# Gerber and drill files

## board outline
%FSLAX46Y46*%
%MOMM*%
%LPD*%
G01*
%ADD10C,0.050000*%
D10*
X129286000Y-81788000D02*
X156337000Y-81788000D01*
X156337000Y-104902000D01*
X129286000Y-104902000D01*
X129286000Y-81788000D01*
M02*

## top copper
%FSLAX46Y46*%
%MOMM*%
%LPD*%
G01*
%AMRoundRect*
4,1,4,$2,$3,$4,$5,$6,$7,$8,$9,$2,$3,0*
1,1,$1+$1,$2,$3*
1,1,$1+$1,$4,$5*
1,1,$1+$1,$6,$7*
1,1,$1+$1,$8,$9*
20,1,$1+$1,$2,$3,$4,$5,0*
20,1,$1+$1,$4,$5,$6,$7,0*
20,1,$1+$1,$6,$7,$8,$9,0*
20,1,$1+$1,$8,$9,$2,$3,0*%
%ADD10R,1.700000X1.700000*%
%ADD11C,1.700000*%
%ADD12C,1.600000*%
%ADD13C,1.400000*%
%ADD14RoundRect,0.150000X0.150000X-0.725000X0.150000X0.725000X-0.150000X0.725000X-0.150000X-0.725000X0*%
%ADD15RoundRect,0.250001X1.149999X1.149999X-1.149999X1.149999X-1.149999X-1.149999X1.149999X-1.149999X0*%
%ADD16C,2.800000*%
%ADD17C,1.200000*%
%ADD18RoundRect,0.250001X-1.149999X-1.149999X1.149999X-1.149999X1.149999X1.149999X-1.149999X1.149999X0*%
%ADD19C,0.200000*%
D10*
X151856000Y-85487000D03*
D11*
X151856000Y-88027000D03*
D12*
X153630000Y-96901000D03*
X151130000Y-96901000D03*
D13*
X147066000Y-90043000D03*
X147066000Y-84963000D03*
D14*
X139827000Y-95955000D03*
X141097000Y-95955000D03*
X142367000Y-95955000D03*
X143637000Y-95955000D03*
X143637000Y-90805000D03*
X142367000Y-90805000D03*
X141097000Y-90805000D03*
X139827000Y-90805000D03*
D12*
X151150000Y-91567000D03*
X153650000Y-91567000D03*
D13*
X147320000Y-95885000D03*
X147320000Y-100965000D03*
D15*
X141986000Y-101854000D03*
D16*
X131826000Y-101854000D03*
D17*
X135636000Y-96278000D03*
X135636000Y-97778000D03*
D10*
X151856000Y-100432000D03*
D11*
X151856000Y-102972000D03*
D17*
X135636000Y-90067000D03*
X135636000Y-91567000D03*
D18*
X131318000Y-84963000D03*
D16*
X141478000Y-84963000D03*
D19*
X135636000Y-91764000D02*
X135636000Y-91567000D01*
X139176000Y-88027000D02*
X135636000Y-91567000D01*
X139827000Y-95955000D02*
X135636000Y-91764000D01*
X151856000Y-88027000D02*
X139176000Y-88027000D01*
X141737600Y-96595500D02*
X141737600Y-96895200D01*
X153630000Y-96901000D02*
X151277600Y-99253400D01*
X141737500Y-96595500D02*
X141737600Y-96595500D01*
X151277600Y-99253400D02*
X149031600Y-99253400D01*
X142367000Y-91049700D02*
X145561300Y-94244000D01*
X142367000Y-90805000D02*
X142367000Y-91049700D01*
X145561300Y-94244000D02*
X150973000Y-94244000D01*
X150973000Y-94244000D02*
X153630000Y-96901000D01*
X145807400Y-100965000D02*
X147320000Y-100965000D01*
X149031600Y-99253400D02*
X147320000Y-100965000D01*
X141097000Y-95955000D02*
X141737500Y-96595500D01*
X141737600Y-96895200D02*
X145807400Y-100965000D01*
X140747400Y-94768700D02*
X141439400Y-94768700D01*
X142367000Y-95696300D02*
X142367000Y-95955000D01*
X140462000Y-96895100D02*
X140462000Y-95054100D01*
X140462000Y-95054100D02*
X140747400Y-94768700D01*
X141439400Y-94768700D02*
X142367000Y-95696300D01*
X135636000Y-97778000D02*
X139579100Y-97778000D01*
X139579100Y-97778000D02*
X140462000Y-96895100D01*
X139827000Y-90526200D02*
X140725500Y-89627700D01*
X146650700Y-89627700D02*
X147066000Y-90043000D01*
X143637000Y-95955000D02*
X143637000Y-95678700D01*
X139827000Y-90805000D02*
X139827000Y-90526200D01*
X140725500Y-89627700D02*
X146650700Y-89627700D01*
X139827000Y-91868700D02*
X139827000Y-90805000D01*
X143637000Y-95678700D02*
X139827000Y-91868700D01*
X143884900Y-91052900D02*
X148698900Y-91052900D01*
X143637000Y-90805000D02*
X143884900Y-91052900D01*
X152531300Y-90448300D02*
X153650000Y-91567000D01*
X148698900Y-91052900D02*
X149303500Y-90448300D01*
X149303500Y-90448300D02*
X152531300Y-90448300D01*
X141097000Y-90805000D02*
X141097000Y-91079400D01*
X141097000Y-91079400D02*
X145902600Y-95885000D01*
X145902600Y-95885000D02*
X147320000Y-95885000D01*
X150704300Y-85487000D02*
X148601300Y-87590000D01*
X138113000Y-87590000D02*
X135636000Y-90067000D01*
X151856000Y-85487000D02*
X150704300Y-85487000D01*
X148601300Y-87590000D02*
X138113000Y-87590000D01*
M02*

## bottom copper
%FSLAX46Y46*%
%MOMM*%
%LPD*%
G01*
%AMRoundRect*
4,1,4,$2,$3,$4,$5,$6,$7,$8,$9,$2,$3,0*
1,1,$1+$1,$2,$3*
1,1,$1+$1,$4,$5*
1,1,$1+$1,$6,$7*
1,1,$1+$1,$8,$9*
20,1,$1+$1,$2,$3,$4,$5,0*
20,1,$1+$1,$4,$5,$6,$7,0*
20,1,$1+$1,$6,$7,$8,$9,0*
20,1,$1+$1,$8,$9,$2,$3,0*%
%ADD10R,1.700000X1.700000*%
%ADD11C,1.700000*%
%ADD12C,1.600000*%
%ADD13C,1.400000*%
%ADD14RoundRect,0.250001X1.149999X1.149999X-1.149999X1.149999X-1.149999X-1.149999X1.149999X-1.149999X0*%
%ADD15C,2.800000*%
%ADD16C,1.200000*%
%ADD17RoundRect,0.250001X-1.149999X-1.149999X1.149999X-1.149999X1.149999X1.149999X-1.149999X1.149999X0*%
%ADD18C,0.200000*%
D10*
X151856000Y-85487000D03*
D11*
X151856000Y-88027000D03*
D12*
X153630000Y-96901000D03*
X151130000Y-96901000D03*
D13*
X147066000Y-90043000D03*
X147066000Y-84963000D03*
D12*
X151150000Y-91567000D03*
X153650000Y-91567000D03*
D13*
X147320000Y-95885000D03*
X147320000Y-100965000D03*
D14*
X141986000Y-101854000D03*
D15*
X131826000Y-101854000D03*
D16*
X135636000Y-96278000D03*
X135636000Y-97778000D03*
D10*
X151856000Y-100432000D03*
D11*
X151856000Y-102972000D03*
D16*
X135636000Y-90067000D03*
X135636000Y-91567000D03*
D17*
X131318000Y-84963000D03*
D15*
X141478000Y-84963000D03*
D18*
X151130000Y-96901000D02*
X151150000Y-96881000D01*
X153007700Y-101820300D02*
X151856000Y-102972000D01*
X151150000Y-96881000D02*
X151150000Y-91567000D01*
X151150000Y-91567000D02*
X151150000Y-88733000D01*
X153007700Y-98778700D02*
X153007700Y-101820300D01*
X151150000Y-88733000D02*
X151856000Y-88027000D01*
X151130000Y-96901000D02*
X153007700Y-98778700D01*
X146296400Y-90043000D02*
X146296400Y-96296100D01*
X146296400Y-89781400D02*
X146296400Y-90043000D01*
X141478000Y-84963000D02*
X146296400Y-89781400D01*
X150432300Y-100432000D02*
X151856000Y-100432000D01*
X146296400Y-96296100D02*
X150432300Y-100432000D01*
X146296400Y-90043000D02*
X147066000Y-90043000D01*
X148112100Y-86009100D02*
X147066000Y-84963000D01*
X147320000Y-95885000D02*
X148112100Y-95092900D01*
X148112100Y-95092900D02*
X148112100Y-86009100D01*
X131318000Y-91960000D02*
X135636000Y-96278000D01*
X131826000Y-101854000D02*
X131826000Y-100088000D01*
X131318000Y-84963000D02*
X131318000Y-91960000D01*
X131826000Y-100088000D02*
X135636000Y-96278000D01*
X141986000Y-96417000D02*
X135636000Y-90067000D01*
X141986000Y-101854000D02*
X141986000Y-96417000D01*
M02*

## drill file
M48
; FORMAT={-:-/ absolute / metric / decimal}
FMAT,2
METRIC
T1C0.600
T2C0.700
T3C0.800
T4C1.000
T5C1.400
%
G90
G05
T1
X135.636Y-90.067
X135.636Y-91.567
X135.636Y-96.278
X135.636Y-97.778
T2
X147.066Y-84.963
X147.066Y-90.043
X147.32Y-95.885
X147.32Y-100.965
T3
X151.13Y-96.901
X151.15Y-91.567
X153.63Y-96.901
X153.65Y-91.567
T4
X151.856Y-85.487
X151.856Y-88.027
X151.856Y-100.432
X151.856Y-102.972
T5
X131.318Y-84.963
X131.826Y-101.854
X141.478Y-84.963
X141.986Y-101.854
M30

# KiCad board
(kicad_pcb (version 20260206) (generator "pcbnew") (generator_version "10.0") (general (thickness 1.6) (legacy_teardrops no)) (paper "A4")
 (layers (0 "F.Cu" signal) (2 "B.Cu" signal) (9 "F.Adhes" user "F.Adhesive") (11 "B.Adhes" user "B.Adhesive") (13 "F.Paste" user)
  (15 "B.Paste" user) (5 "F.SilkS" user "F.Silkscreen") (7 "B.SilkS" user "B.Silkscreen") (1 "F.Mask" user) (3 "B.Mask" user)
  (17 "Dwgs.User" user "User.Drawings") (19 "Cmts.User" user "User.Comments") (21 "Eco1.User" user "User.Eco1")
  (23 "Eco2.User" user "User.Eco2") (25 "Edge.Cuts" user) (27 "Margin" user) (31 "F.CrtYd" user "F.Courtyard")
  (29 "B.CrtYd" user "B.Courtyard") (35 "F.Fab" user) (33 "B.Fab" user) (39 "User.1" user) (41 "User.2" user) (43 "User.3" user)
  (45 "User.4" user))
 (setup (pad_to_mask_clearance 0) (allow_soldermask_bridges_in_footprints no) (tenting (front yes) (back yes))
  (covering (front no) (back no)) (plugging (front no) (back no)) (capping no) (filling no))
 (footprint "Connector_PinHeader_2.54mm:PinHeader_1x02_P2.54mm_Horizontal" (layer "F.Cu") (at 151.856 85.487)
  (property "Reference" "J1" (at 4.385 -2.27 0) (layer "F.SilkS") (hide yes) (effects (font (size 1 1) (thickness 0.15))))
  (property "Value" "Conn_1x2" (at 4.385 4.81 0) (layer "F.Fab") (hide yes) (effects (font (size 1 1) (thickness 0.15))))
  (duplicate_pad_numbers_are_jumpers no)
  (pad "1" thru_hole rect (at 0 0) (size 1.7 1.7) (drill 1) (layers "*.Cu" "*.Mask") (remove_unused_layers no) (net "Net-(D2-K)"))
  (pad "2" thru_hole circle (at 0 2.54) (size 1.7 1.7) (drill 1) (layers "*.Cu" "*.Mask") (remove_unused_layers no) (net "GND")))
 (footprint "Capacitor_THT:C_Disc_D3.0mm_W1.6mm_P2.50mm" (layer "F.Cu") (at 153.63 96.901 180)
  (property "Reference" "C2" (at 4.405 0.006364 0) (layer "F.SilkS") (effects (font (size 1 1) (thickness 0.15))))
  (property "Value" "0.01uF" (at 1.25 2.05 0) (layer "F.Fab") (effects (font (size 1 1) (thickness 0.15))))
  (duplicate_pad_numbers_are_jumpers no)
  (pad "1" thru_hole circle (at 0 0 180) (size 1.6 1.6) (drill 0.8) (layers "*.Cu" "*.Mask") (remove_unused_layers no)
   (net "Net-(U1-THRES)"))
  (pad "2" thru_hole circle (at 2.5 0 180) (size 1.6 1.6) (drill 0.8) (layers "*.Cu" "*.Mask") (remove_unused_layers no) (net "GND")))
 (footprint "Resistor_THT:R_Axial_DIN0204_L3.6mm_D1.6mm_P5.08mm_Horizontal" (layer "F.Cu") (at 147.066 90.043 90)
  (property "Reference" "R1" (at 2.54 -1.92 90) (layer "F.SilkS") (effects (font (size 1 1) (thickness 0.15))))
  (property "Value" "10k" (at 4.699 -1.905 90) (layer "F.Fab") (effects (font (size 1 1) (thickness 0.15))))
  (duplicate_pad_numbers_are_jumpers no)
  (pad "1" thru_hole circle (at 0 0 90) (size 1.4 1.4) (drill 0.7) (layers "*.Cu" "*.Mask") (remove_unused_layers no) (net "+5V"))
  (pad "2" thru_hole circle (at 5.08 0 90) (size 1.4 1.4) (drill 0.7) (layers "*.Cu" "*.Mask") (remove_unused_layers no)
   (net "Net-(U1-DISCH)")))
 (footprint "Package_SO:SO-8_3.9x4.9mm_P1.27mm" (layer "F.Cu") (at 141.732 93.38 90)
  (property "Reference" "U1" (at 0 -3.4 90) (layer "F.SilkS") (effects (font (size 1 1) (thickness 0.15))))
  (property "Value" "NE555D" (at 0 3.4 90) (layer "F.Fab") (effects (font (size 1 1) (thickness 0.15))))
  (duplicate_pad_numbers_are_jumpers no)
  (pad "1" smd roundrect (at -2.575 -1.905 90) (size 1.75 0.6) (layers "F.Cu" "F.Mask" "F.Paste") (roundrect_rratio 0.25) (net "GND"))
  (pad "2" smd roundrect (at -2.575 -0.635 90) (size 1.75 0.6) (layers "F.Cu" "F.Mask" "F.Paste") (roundrect_rratio 0.25)
   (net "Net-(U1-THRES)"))
  (pad "3" smd roundrect (at -2.575 0.635 90) (size 1.75 0.6) (layers "F.Cu" "F.Mask" "F.Paste") (roundrect_rratio 0.25)
   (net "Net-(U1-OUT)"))
  (pad "4" smd roundrect (at -2.575 1.905 90) (size 1.75 0.6) (layers "F.Cu" "F.Mask" "F.Paste") (roundrect_rratio 0.25) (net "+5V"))
  (pad "5" smd roundrect (at 2.575 1.905 90) (size 1.75 0.6) (layers "F.Cu" "F.Mask" "F.Paste") (roundrect_rratio 0.25)
   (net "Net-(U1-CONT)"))
  (pad "6" smd roundrect (at 2.575 0.635 90) (size 1.75 0.6) (layers "F.Cu" "F.Mask" "F.Paste") (roundrect_rratio 0.25)
   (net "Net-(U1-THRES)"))
  (pad "7" smd roundrect (at 2.575 -0.635 90) (size 1.75 0.6) (layers "F.Cu" "F.Mask" "F.Paste") (roundrect_rratio 0.25)
   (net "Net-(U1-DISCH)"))
  (pad "8" smd roundrect (at 2.575 -1.905 90) (size 1.75 0.6) (layers "F.Cu" "F.Mask" "F.Paste") (roundrect_rratio 0.25) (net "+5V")))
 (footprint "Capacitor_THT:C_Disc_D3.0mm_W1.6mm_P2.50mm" (layer "F.Cu") (at 151.15 91.567)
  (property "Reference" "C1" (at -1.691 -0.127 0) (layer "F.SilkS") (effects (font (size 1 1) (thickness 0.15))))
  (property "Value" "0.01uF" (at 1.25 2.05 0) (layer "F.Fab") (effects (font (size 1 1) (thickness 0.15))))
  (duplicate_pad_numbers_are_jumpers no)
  (pad "1" thru_hole circle (at 0 0) (size 1.6 1.6) (drill 0.8) (layers "*.Cu" "*.Mask") (remove_unused_layers no) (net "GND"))
  (pad "2" thru_hole circle (at 2.5 0) (size 1.6 1.6) (drill 0.8) (layers "*.Cu" "*.Mask") (remove_unused_layers no) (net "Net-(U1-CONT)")))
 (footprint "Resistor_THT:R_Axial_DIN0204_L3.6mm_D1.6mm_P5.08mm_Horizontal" (layer "F.Cu") (at 147.32 95.885 -90)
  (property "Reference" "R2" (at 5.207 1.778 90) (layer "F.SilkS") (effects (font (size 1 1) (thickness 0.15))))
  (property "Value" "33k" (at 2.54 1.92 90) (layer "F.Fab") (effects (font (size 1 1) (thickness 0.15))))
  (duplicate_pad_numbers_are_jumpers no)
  (pad "1" thru_hole circle (at 0 0 270) (size 1.4 1.4) (drill 0.7) (layers "*.Cu" "*.Mask") (remove_unused_layers no)
   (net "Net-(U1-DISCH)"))
  (pad "2" thru_hole circle (at 5.08 0 270) (size 1.4 1.4) (drill 0.7) (layers "*.Cu" "*.Mask") (remove_unused_layers no)
   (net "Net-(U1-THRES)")))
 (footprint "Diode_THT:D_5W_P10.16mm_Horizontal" (layer "F.Cu") (at 141.986 101.854 180)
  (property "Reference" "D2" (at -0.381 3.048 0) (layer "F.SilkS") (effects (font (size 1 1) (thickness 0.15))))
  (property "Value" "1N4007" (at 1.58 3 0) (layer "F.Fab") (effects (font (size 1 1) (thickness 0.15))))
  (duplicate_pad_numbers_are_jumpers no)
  (pad "1" thru_hole roundrect (at 0 0 180) (size 2.8 2.8) (drill 1.4) (layers "*.Cu" "*.Mask") (remove_unused_layers no)
   (roundrect_rratio 0.089286) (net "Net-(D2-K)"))
  (pad "2" thru_hole circle (at 10.16 0 180) (size 2.8 2.8) (drill 1.4) (layers "*.Cu" "*.Mask") (remove_unused_layers no)
   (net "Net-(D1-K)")))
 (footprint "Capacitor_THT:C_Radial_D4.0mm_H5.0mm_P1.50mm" (layer "F.Cu") (at 135.636 96.278 -90)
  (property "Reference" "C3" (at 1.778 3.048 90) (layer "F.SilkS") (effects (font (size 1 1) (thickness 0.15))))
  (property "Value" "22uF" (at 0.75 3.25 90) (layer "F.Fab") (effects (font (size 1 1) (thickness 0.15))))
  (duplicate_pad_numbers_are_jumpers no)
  (pad "1" thru_hole circle (at 0 0 270) (size 1.2 1.2) (drill 0.6) (layers "*.Cu" "*.Mask") (remove_unused_layers no) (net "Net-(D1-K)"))
  (pad "2" thru_hole circle (at 1.5 0 270) (size 1.2 1.2) (drill 0.6) (layers "*.Cu" "*.Mask") (remove_unused_layers no)
   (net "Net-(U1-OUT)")))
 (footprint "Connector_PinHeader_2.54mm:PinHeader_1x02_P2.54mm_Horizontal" (layer "F.Cu") (at 151.856 100.432)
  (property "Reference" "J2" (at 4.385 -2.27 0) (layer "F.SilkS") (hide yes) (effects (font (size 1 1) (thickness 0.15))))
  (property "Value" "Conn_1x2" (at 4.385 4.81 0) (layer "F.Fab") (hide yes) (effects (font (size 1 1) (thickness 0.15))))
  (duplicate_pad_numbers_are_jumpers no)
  (pad "1" thru_hole rect (at 0 0) (size 1.7 1.7) (drill 1) (layers "*.Cu" "*.Mask") (remove_unused_layers no) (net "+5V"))
  (pad "2" thru_hole circle (at 0 2.54) (size 1.7 1.7) (drill 1) (layers "*.Cu" "*.Mask") (remove_unused_layers no) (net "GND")))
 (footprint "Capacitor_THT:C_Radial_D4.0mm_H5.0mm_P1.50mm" (layer "F.Cu") (at 135.636 90.067 -90)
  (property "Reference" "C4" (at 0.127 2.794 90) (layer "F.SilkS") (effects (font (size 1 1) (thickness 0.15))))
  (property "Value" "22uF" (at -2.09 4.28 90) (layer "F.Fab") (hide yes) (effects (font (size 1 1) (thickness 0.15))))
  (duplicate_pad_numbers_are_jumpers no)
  (pad "1" thru_hole circle (at 0 0 270) (size 1.2 1.2) (drill 0.6) (layers "*.Cu" "*.Mask") (remove_unused_layers no) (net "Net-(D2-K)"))
  (pad "2" thru_hole circle (at 1.5 0 270) (size 1.2 1.2) (drill 0.6) (layers "*.Cu" "*.Mask") (remove_unused_layers no) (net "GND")))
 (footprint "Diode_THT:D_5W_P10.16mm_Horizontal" (layer "F.Cu") (at 131.318 84.963)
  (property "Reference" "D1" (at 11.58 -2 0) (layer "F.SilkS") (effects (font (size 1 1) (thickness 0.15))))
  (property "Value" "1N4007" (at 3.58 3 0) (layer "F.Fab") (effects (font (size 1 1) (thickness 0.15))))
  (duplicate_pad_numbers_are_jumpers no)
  (pad "1" thru_hole roundrect (at 0 0) (size 2.8 2.8) (drill 1.4) (layers "*.Cu" "*.Mask") (remove_unused_layers no)
   (roundrect_rratio 0.089286) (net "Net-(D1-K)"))
  (pad "2" thru_hole circle (at 10.16 0) (size 2.8 2.8) (drill 1.4) (layers "*.Cu" "*.Mask") (remove_unused_layers no) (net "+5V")))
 (gr_rect (start 129.286 81.788) (end 156.337 104.902) (stroke (width 0.05) (type default)) (fill no) (layer "Edge.Cuts"))
 (segment (start 135.636 91.764) (end 135.636 91.567) (width 0.2) (layer "F.Cu") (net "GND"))
 (segment (start 139.176 88.027) (end 135.636 91.567) (width 0.2) (layer "F.Cu") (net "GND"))
 (segment (start 139.827 95.955) (end 135.636 91.764) (width 0.2) (layer "F.Cu") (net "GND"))
 (segment (start 151.856 88.027) (end 139.176 88.027) (width 0.2) (layer "F.Cu") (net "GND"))
 (segment (start 151.13 96.901) (end 151.15 96.881) (width 0.2) (layer "B.Cu") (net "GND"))
 (segment (start 153.0077 101.8203) (end 151.856 102.972) (width 0.2) (layer "B.Cu") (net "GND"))
 (segment (start 151.15 96.881) (end 151.15 91.567) (width 0.2) (layer "B.Cu") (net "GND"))
 (segment (start 151.15 91.567) (end 151.15 88.733) (width 0.2) (layer "B.Cu") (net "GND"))
 (segment (start 153.0077 98.7787) (end 153.0077 101.8203) (width 0.2) (layer "B.Cu") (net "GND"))
 (segment (start 151.15 88.733) (end 151.856 88.027) (width 0.2) (layer "B.Cu") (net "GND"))
 (segment (start 151.13 96.901) (end 153.0077 98.7787) (width 0.2) (layer "B.Cu") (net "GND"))
 (segment (start 141.7376 96.5955) (end 141.7376 96.8952) (width 0.2) (layer "F.Cu") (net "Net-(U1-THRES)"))
 (segment (start 153.63 96.901) (end 151.2776 99.2534) (width 0.2) (layer "F.Cu") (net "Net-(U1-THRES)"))
 (segment (start 141.7375 96.5955) (end 141.7376 96.5955) (width 0.2) (layer "F.Cu") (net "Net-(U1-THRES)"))
 (segment (start 151.2776 99.2534) (end 149.0316 99.2534) (width 0.2) (layer "F.Cu") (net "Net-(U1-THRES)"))
 (segment (start 142.367 91.0497) (end 145.5613 94.244) (width 0.2) (layer "F.Cu") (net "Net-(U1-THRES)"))
 (segment (start 142.367 90.805) (end 142.367 91.0497) (width 0.2) (layer "F.Cu") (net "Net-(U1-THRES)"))
 (segment (start 145.5613 94.244) (end 150.973 94.244) (width 0.2) (layer "F.Cu") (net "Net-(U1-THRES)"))
 (segment (start 150.973 94.244) (end 153.63 96.901) (width 0.2) (layer "F.Cu") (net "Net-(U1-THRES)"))
 (segment (start 145.8074 100.965) (end 147.32 100.965) (width 0.2) (layer "F.Cu") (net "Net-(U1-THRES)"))
 (segment (start 149.0316 99.2534) (end 147.32 100.965) (width 0.2) (layer "F.Cu") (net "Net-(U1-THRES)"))
 (segment (start 141.097 95.955) (end 141.7375 96.5955) (width 0.2) (layer "F.Cu") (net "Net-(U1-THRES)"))
 (segment (start 141.7376 96.8952) (end 145.8074 100.965) (width 0.2) (layer "F.Cu") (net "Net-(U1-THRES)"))
 (segment (start 140.7474 94.7687) (end 141.4394 94.7687) (width 0.2) (layer "F.Cu") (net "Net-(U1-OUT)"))
 (segment (start 142.367 95.6963) (end 142.367 95.955) (width 0.2) (layer "F.Cu") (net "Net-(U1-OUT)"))
 (segment (start 140.462 96.8951) (end 140.462 95.0541) (width 0.2) (layer "F.Cu") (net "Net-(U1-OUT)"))
 (segment (start 140.462 95.0541) (end 140.7474 94.7687) (width 0.2) (layer "F.Cu") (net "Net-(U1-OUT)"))
 (segment (start 141.4394 94.7687) (end 142.367 95.6963) (width 0.2) (layer "F.Cu") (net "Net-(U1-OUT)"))
 (segment (start 135.636 97.778) (end 139.5791 97.778) (width 0.2) (layer "F.Cu") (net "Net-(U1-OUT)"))
 (segment (start 139.5791 97.778) (end 140.462 96.8951) (width 0.2) (layer "F.Cu") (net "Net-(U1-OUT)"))
 (segment (start 139.827 90.5262) (end 140.7255 89.6277) (width 0.2) (layer "F.Cu") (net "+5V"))
 (segment (start 146.6507 89.6277) (end 147.066 90.043) (width 0.2) (layer "F.Cu") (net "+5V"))
 (segment (start 143.637 95.955) (end 143.637 95.6787) (width 0.2) (layer "F.Cu") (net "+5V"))
 (segment (start 139.827 90.805) (end 139.827 90.5262) (width 0.2) (layer "F.Cu") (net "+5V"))
 (segment (start 140.7255 89.6277) (end 146.6507 89.6277) (width 0.2) (layer "F.Cu") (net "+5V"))
 (segment (start 139.827 91.8687) (end 139.827 90.805) (width 0.2) (layer "F.Cu") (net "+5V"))
 (segment (start 143.637 95.6787) (end 139.827 91.8687) (width 0.2) (layer "F.Cu") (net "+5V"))
 (segment (start 146.2964 90.043) (end 146.2964 96.2961) (width 0.2) (layer "B.Cu") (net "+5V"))
 (segment (start 146.2964 89.7814) (end 146.2964 90.043) (width 0.2) (layer "B.Cu") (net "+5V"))
 (segment (start 141.478 84.963) (end 146.2964 89.7814) (width 0.2) (layer "B.Cu") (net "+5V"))
 (segment (start 150.4323 100.432) (end 151.856 100.432) (width 0.2) (layer "B.Cu") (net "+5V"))
 (segment (start 146.2964 96.2961) (end 150.4323 100.432) (width 0.2) (layer "B.Cu") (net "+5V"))
 (segment (start 146.2964 90.043) (end 147.066 90.043) (width 0.2) (layer "B.Cu") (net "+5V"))
 (segment (start 143.8849 91.0529) (end 148.6989 91.0529) (width 0.2) (layer "F.Cu") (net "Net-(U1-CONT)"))
 (segment (start 143.637 90.805) (end 143.8849 91.0529) (width 0.2) (layer "F.Cu") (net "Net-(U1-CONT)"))
 (segment (start 152.5313 90.4483) (end 153.65 91.567) (width 0.2) (layer "F.Cu") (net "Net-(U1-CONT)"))
 (segment (start 148.6989 91.0529) (end 149.3035 90.4483) (width 0.2) (layer "F.Cu") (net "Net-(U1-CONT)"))
 (segment (start 149.3035 90.4483) (end 152.5313 90.4483) (width 0.2) (layer "F.Cu") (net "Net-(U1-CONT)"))
 (segment (start 141.097 90.805) (end 141.097 91.0794) (width 0.2) (layer "F.Cu") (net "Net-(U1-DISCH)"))
 (segment (start 141.097 91.0794) (end 145.9026 95.885) (width 0.2) (layer "F.Cu") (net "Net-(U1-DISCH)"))
 (segment (start 145.9026 95.885) (end 147.32 95.885) (width 0.2) (layer "F.Cu") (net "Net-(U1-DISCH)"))
 (segment (start 148.1121 86.0091) (end 147.066 84.963) (width 0.2) (layer "B.Cu") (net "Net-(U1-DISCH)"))
 (segment (start 147.32 95.885) (end 148.1121 95.0929) (width 0.2) (layer "B.Cu") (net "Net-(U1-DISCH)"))
 (segment (start 148.1121 95.0929) (end 148.1121 86.0091) (width 0.2) (layer "B.Cu") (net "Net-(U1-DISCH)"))
 (segment (start 131.318 91.96) (end 135.636 96.278) (width 0.2) (layer "B.Cu") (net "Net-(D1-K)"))
 (segment (start 131.826 101.854) (end 131.826 100.088) (width 0.2) (layer "B.Cu") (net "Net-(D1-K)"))
 (segment (start 131.318 84.963) (end 131.318 91.96) (width 0.2) (layer "B.Cu") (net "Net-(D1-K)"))
 (segment (start 131.826 100.088) (end 135.636 96.278) (width 0.2) (layer "B.Cu") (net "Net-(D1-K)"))
 (segment (start 150.7043 85.487) (end 148.6013 87.59) (width 0.2) (layer "F.Cu") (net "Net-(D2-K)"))
 (segment (start 138.113 87.59) (end 135.636 90.067) (width 0.2) (layer "F.Cu") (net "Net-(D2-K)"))
 (segment (start 151.856 85.487) (end 150.7043 85.487) (width 0.2) (layer "F.Cu") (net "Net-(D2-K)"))
 (segment (start 148.6013 87.59) (end 138.113 87.59) (width 0.2) (layer "F.Cu") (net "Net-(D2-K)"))
 (segment (start 141.986 96.417) (end 135.636 90.067) (width 0.2) (layer "B.Cu") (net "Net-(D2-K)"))
 (segment (start 141.986 101.854) (end 141.986 96.417) (width 0.2) (layer "B.Cu") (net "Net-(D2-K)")))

